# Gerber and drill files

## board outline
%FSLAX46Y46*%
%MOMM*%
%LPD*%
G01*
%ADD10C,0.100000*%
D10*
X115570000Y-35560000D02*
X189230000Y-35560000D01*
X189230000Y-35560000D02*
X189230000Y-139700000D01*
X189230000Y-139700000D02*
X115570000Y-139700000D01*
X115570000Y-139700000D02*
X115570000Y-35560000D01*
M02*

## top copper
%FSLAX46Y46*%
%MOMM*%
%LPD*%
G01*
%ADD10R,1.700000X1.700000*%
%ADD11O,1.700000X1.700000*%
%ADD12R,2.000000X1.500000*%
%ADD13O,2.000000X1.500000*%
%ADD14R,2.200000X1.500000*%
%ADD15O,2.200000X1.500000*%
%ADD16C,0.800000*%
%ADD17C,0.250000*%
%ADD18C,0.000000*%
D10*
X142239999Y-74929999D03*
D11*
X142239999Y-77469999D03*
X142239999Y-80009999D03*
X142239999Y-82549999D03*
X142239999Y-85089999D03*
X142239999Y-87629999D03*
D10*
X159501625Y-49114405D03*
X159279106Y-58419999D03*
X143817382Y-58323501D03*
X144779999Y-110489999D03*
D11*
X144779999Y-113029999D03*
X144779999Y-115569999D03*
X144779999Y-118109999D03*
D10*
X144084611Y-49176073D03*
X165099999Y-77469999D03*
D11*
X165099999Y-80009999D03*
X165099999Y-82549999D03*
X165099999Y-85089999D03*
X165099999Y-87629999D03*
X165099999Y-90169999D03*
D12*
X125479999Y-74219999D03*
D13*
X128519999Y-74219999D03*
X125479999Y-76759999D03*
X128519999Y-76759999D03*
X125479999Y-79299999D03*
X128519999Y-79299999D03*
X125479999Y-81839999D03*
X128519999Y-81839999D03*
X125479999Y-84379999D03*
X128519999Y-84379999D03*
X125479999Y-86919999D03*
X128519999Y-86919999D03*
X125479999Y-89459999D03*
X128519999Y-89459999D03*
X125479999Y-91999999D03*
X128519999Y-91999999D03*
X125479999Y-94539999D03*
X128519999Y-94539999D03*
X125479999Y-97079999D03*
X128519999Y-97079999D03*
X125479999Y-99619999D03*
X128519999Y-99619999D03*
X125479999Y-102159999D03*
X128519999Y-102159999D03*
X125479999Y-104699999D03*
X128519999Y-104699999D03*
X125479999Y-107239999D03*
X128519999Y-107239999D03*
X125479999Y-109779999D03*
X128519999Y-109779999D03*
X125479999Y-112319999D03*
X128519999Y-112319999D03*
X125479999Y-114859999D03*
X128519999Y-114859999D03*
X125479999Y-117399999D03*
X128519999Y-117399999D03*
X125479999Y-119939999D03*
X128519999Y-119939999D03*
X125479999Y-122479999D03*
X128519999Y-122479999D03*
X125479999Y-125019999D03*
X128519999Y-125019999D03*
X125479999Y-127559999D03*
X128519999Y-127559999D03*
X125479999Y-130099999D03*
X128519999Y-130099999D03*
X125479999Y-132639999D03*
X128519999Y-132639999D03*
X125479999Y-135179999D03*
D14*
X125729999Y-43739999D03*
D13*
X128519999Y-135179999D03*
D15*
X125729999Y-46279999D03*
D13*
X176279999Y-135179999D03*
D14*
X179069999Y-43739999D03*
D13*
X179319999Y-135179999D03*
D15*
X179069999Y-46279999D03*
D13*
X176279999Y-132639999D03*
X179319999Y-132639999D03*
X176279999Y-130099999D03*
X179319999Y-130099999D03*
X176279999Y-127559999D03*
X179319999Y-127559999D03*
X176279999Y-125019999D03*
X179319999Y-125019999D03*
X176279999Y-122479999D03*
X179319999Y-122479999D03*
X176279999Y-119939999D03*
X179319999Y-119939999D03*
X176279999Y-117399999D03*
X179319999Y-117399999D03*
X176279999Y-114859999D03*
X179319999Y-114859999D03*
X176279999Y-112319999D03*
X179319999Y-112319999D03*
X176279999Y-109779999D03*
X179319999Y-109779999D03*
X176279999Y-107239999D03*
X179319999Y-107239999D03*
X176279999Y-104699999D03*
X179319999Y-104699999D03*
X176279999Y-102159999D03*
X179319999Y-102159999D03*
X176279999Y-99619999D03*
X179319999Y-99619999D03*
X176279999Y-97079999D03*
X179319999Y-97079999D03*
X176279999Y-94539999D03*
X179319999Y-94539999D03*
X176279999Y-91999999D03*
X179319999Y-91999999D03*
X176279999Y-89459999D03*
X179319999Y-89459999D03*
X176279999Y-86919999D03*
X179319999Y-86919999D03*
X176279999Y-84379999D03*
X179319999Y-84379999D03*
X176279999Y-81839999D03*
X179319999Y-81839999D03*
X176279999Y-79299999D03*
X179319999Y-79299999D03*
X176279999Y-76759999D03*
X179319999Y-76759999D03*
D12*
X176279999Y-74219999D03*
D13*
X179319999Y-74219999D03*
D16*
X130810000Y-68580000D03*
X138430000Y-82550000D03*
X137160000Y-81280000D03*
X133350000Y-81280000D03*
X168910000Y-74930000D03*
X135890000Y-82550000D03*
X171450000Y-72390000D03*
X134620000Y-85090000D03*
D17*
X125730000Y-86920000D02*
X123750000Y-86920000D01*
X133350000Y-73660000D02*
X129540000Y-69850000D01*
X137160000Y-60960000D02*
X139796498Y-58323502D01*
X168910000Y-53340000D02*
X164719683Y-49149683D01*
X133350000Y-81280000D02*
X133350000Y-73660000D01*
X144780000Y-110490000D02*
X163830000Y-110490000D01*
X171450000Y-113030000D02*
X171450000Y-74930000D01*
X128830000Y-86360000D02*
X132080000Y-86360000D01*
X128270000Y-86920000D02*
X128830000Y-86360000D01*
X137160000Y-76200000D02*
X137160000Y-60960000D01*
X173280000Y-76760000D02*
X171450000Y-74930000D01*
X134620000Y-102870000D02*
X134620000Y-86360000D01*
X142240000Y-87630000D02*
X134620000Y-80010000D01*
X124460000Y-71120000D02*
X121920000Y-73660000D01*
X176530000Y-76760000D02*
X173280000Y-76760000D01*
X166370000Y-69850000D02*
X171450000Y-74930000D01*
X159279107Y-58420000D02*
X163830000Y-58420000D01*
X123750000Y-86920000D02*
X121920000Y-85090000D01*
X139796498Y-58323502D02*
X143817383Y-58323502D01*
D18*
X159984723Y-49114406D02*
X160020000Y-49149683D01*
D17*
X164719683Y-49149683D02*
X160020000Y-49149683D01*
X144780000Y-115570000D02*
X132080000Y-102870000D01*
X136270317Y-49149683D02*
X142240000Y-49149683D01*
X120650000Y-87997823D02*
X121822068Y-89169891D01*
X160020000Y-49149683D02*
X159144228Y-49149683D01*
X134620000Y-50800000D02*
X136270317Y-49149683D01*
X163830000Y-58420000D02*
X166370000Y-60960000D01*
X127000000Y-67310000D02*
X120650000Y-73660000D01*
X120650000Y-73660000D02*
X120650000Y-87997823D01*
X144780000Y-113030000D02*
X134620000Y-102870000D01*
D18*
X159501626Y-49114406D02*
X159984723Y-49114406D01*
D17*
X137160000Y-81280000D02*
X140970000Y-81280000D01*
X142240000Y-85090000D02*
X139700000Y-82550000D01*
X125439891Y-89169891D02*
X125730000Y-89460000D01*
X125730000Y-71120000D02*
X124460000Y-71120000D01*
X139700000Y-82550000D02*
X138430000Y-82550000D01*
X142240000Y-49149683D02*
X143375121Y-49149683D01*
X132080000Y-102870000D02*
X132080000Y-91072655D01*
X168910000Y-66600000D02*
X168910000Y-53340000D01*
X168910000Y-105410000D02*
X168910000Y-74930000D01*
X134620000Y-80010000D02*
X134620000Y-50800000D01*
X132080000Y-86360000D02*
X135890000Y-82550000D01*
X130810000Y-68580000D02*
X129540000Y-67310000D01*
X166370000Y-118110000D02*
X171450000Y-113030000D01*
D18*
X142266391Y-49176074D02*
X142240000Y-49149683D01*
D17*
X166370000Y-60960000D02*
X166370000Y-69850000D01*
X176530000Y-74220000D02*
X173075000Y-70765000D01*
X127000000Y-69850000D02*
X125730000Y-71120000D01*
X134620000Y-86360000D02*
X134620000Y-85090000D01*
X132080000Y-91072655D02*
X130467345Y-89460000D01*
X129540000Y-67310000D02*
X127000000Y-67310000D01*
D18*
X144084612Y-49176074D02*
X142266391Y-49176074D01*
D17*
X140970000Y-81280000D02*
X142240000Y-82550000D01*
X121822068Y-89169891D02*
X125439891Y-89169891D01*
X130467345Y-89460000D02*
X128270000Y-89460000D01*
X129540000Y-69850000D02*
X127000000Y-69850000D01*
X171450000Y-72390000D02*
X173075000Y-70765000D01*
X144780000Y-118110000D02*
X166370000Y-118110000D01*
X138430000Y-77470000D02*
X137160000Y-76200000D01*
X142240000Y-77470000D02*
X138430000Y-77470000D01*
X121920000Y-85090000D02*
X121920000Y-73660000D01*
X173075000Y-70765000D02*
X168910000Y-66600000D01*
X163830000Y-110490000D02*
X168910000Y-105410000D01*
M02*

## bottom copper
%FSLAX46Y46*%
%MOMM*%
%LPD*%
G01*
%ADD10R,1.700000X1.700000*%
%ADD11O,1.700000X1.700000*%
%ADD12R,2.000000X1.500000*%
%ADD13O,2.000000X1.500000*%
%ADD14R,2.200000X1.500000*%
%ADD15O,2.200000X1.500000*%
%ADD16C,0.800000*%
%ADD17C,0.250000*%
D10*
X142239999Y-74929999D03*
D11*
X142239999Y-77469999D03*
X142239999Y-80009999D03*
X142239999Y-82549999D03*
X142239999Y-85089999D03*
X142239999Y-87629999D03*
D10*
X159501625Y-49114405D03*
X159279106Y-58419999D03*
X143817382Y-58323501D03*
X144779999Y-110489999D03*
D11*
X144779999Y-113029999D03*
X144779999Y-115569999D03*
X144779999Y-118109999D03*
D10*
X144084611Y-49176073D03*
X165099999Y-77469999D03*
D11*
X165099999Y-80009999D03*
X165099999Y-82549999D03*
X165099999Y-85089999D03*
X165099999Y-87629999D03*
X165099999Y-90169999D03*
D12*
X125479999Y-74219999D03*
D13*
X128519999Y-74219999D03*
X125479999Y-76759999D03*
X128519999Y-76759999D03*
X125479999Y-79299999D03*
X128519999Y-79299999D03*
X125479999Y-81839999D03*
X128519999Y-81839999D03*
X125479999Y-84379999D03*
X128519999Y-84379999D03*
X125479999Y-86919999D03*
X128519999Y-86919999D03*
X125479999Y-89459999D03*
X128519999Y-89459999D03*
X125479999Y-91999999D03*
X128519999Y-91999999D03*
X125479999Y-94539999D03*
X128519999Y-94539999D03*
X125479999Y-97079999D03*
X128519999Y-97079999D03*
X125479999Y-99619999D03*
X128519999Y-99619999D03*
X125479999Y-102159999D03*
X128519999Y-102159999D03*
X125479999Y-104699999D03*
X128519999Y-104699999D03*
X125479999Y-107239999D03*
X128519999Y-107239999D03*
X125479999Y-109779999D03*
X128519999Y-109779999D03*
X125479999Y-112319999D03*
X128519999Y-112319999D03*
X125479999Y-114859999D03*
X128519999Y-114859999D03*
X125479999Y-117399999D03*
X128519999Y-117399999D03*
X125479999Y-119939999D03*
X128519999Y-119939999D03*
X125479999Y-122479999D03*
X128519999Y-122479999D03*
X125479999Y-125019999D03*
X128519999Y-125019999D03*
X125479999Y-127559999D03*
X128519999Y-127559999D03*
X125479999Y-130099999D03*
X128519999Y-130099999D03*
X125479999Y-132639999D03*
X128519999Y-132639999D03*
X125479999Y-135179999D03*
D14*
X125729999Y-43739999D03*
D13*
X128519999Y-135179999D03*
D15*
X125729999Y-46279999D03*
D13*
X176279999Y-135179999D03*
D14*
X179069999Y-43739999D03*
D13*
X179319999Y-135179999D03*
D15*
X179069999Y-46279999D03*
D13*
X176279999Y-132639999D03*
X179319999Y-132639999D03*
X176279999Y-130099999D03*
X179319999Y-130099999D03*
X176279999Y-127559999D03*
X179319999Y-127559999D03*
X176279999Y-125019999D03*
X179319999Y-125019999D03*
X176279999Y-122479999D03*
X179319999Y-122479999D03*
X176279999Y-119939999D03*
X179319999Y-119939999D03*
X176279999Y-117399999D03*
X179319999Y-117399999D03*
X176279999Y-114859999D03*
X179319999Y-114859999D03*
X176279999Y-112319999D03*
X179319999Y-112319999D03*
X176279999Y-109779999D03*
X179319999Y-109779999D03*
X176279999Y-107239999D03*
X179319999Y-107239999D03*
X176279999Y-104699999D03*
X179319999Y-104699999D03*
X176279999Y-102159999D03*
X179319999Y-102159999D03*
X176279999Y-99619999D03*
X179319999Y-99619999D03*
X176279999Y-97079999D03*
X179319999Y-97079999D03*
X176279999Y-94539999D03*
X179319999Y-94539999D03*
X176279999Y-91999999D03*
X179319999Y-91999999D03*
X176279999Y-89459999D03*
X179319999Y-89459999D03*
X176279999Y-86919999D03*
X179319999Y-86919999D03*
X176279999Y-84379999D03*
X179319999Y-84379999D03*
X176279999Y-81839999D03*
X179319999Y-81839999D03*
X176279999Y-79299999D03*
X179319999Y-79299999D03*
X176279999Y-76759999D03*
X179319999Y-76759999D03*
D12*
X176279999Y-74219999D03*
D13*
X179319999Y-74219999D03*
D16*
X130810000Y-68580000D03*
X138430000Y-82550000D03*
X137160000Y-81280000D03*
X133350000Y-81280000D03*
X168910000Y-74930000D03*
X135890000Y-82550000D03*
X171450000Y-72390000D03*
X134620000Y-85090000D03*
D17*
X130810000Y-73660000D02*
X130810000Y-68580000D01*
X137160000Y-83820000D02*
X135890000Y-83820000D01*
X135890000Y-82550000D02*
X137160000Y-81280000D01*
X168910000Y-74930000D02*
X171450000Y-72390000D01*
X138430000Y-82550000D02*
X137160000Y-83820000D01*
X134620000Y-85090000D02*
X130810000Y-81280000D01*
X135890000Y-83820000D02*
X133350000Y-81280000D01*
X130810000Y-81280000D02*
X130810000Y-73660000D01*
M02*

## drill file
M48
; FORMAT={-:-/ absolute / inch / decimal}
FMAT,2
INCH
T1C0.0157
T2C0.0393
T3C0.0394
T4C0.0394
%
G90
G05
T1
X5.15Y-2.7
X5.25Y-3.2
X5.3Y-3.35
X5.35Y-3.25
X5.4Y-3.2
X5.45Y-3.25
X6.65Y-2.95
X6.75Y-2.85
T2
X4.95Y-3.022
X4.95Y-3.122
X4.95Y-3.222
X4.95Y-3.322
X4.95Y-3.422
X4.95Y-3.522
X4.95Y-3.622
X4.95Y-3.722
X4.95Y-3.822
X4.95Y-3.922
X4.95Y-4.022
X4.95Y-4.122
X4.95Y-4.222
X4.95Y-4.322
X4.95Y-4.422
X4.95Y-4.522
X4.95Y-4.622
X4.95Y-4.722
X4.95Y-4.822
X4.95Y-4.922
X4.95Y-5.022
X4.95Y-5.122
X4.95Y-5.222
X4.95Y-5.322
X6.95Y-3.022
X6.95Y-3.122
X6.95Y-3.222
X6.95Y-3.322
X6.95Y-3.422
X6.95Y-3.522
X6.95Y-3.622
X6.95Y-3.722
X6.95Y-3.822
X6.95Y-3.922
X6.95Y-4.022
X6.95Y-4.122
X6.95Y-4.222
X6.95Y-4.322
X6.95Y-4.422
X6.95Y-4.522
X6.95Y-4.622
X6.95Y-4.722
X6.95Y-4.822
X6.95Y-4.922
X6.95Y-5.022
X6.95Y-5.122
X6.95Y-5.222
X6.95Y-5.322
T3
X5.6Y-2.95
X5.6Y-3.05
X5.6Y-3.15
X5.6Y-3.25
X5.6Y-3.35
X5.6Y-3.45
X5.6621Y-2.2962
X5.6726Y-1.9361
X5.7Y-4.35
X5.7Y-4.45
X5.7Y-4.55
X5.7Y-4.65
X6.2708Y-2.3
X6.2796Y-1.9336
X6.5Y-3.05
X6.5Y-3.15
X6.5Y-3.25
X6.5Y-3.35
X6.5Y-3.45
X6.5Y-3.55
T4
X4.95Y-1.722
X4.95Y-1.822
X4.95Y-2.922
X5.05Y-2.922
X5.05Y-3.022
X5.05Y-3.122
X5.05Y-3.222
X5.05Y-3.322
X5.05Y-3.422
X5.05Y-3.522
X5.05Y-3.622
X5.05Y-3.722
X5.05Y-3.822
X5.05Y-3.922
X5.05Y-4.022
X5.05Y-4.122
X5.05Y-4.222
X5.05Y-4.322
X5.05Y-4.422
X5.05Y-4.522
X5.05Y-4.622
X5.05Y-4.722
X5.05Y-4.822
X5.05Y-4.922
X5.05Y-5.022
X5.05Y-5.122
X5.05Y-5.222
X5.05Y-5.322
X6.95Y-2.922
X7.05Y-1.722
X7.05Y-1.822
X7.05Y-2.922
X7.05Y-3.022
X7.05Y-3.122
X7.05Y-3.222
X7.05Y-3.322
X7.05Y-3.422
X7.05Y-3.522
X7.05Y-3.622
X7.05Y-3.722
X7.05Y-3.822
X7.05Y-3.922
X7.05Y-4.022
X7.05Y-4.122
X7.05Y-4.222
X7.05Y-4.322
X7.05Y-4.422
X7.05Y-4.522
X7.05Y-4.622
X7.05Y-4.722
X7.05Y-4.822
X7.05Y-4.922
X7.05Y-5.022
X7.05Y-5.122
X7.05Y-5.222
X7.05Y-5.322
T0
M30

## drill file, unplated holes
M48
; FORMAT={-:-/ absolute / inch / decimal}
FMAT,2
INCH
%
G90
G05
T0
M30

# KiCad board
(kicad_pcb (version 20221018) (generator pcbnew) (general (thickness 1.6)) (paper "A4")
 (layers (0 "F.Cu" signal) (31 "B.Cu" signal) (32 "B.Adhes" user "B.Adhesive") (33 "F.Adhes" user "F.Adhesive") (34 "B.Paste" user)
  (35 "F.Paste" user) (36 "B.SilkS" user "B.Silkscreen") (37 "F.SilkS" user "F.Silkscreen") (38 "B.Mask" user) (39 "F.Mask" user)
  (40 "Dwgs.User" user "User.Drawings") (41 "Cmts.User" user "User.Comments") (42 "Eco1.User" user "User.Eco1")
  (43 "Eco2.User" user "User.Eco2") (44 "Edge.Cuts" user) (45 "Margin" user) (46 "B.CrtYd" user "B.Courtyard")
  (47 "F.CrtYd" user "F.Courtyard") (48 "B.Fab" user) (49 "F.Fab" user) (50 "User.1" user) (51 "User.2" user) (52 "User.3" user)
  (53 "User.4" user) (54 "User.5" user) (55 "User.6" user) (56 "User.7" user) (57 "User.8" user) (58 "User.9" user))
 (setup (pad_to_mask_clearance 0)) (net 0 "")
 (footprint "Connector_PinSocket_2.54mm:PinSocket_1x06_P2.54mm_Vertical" (layer "F.Cu") (at 142.24 74.93)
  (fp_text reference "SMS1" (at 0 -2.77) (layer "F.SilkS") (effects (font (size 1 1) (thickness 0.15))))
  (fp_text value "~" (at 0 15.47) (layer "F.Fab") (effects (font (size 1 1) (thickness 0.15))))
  (pad "1" thru_hole rect (at 0 0) (size 1.7 1.7) (drill 1) (layers "*.Cu" "*.Mask"))
  (pad "2" thru_hole oval (at 0 2.54) (size 1.7 1.7) (drill 1) (layers "*.Cu" "*.Mask"))
  (pad "3" thru_hole oval (at 0 5.08) (size 1.7 1.7) (drill 1) (layers "*.Cu" "*.Mask"))
  (pad "4" thru_hole oval (at 0 7.62) (size 1.7 1.7) (drill 1) (layers "*.Cu" "*.Mask"))
  (pad "5" thru_hole oval (at 0 10.16) (size 1.7 1.7) (drill 1) (layers "*.Cu" "*.Mask"))
  (pad "6" thru_hole oval (at 0 12.7) (size 1.7 1.7) (drill 1) (layers "*.Cu" "*.Mask")))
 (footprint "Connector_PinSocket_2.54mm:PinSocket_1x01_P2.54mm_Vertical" (layer "F.Cu") (at 159.501626 49.114406 180)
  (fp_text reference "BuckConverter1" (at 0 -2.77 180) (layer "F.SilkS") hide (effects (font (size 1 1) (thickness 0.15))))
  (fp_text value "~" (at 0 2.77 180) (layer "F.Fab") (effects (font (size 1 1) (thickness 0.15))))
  (pad "1" thru_hole rect (at 0 0 180) (size 1.7 1.7) (drill 1) (layers "*.Cu" "*.Mask")))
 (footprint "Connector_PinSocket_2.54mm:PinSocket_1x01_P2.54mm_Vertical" (layer "F.Cu") (at 159.279107 58.42 180)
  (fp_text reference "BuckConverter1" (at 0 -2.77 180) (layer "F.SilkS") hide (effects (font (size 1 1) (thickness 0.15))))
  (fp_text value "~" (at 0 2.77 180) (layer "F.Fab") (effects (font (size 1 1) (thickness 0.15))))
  (pad "1" thru_hole rect (at 0 0 180) (size 1.7 1.7) (drill 1) (layers "*.Cu" "*.Mask")))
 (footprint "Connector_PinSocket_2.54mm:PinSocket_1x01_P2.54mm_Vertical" (layer "F.Cu") (at 143.817383 58.323502 180)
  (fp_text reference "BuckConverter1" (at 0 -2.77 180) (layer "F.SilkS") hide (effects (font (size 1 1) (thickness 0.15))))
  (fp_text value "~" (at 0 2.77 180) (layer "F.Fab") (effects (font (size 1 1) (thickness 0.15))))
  (pad "1" thru_hole rect (at 0 0 180) (size 1.7 1.7) (drill 1) (layers "*.Cu" "*.Mask")))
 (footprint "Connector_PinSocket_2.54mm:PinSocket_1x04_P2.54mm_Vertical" (layer "F.Cu") (at 144.78 110.49)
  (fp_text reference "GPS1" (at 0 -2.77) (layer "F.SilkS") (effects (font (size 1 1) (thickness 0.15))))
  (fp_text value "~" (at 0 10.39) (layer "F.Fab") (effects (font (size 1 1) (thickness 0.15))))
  (pad "1" thru_hole rect (at 0 0) (size 1.7 1.7) (drill 1) (layers "*.Cu" "*.Mask"))
  (pad "2" thru_hole oval (at 0 2.54) (size 1.7 1.7) (drill 1) (layers "*.Cu" "*.Mask"))
  (pad "3" thru_hole oval (at 0 5.08) (size 1.7 1.7) (drill 1) (layers "*.Cu" "*.Mask"))
  (pad "4" thru_hole oval (at 0 7.62) (size 1.7 1.7) (drill 1) (layers "*.Cu" "*.Mask")))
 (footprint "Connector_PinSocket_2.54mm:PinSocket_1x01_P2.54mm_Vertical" (layer "F.Cu") (at 144.084612 49.176074 180)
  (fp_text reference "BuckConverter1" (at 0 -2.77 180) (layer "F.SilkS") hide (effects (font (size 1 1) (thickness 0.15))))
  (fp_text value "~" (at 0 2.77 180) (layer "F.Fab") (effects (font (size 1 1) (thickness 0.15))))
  (pad "1" thru_hole rect (at 0 0 180) (size 1.7 1.7) (drill 1) (layers "*.Cu" "*.Mask")))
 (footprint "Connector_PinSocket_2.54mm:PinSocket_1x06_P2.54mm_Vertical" (layer "F.Cu") (at 165.1 77.47)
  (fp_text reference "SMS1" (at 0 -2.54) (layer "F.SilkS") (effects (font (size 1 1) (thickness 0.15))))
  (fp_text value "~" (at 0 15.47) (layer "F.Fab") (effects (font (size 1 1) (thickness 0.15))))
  (pad "1" thru_hole rect (at 0 0) (size 1.7 1.7) (drill 1) (layers "*.Cu" "*.Mask"))
  (pad "2" thru_hole oval (at 0 2.54) (size 1.7 1.7) (drill 1) (layers "*.Cu" "*.Mask"))
  (pad "3" thru_hole oval (at 0 5.08) (size 1.7 1.7) (drill 1) (layers "*.Cu" "*.Mask"))
  (pad "4" thru_hole oval (at 0 7.62) (size 1.7 1.7) (drill 1) (layers "*.Cu" "*.Mask"))
  (pad "5" thru_hole oval (at 0 10.16) (size 1.7 1.7) (drill 1) (layers "*.Cu" "*.Mask"))
  (pad "6" thru_hole oval (at 0 12.7) (size 1.7 1.7) (drill 1) (layers "*.Cu" "*.Mask")))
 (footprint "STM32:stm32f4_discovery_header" (layer "F.Cu") (at 152.4 88.9 90)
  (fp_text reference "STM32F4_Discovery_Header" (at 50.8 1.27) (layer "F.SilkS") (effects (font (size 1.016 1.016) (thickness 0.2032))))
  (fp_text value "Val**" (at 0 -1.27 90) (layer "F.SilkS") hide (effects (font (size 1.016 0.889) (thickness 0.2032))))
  (pad "1" thru_hole rect (at 14.68 -26.67 90) (size 1.5 2) (drill 1.00076 (offset 0 -0.25)) (layers "*.Cu" "*.Mask" "F.SilkS"))
  (pad "2" thru_hole oval (at 14.68 -24.13 90) (size 1.5 2) (drill 1.00076 (offset 0 0.25)) (layers "*.Cu" "*.Mask" "F.SilkS"))
  (pad "3" thru_hole oval (at 12.14 -26.67 90) (size 1.5 2) (drill 0.99822 (offset 0 -0.25)) (layers "*.Cu" "*.Mask" "F.SilkS"))
  (pad "4" thru_hole oval (at 12.14 -24.13 90) (size 1.5 2) (drill 1.00076 (offset 0 0.25)) (layers "*.Cu" "*.Mask" "F.SilkS"))
  (pad "5" thru_hole oval (at 9.6 -26.67 90) (size 1.5 2) (drill 0.99822 (offset 0 -0.25)) (layers "*.Cu" "*.Mask" "F.SilkS"))
  (pad "6" thru_hole oval (at 9.6 -24.13 90) (size 1.5 2) (drill 1.00076 (offset 0 0.25)) (layers "*.Cu" "*.Mask" "F.SilkS"))
  (pad "7" thru_hole oval (at 7.06 -26.67 90) (size 1.5 2) (drill 0.99822 (offset 0 -0.25)) (layers "*.Cu" "*.Mask" "F.SilkS"))
  (pad "8" thru_hole oval (at 7.06 -24.13 90) (size 1.5 2) (drill 1.00076 (offset 0 0.25)) (layers "*.Cu" "*.Mask" "F.SilkS"))
  (pad "9" thru_hole oval (at 4.52 -26.67 90) (size 1.5 2) (drill 0.99822 (offset 0 -0.25)) (layers "*.Cu" "*.Mask" "F.SilkS"))
  (pad "10" thru_hole oval (at 4.52 -24.13 90) (size 1.5 2) (drill 1.00076 (offset 0 0.25)) (layers "*.Cu" "*.Mask" "F.SilkS"))
  (pad "11" thru_hole oval (at 1.98 -26.67 90) (size 1.5 2) (drill 0.99822 (offset 0 -0.25)) (layers "*.Cu" "*.Mask" "F.SilkS"))
  (pad "12" thru_hole oval (at 1.98 -24.13 90) (size 1.5 2) (drill 1.00076 (offset 0 0.25)) (layers "*.Cu" "*.Mask" "F.SilkS"))
  (pad "13" thru_hole oval (at -0.56 -26.67 90) (size 1.5 2) (drill 0.99822 (offset 0 -0.25)) (layers "*.Cu" "*.Mask" "F.SilkS"))
  (pad "14" thru_hole oval (at -0.56 -24.13 90) (size 1.5 2) (drill 1.00076 (offset 0 0.25)) (layers "*.Cu" "*.Mask" "F.SilkS"))
  (pad "15" thru_hole oval (at -3.1 -26.67 90) (size 1.5 2) (drill 0.99822 (offset 0 -0.25)) (layers "*.Cu" "*.Mask" "F.SilkS"))
  (pad "16" thru_hole oval (at -3.1 -24.13 90) (size 1.5 2) (drill 1.00076 (offset 0 0.25)) (layers "*.Cu" "*.Mask" "F.SilkS"))
  (pad "17" thru_hole oval (at -5.64 -26.67 90) (size 1.5 2) (drill 0.99822 (offset 0 -0.25)) (layers "*.Cu" "*.Mask" "F.SilkS"))
  (pad "18" thru_hole oval (at -5.64 -24.13 90) (size 1.5 2) (drill 1.00076 (offset 0 0.25)) (layers "*.Cu" "*.Mask" "F.SilkS"))
  (pad "19" thru_hole oval (at -8.18 -26.67 90) (size 1.5 2) (drill 0.99822 (offset 0 -0.25)) (layers "*.Cu" "*.Mask" "F.SilkS"))
  (pad "20" thru_hole oval (at -8.18 -24.13 90) (size 1.5 2) (drill 1.00076 (offset 0 0.25)) (layers "*.Cu" "*.Mask" "F.SilkS"))
  (pad "21" thru_hole oval (at -10.72 -26.67 90) (size 1.5 2) (drill 0.99822 (offset 0 -0.25)) (layers "*.Cu" "*.Mask" "F.SilkS"))
  (pad "22" thru_hole oval (at -10.72 -24.13 90) (size 1.5 2) (drill 1.00076 (offset 0 0.25)) (layers "*.Cu" "*.Mask" "F.SilkS"))
  (pad "23" thru_hole oval (at -13.26 -26.67 90) (size 1.5 2) (drill 0.99822 (offset 0 -0.25)) (layers "*.Cu" "*.Mask" "F.SilkS"))
  (pad "24" thru_hole oval (at -13.26 -24.13 90) (size 1.5 2) (drill 1.00076 (offset 0 0.25)) (layers "*.Cu" "*.Mask" "F.SilkS"))
  (pad "25" thru_hole oval (at -15.8 -26.67 90) (size 1.5 2) (drill 0.99822 (offset 0 -0.25)) (layers "*.Cu" "*.Mask" "F.SilkS"))
  (pad "26" thru_hole oval (at -15.8 -24.13 90) (size 1.5 2) (drill 1.00076 (offset 0 0.25)) (layers "*.Cu" "*.Mask" "F.SilkS"))
  (pad "27" thru_hole oval (at -18.34 -26.67 90) (size 1.5 2) (drill 0.99822 (offset 0 -0.25)) (layers "*.Cu" "*.Mask" "F.SilkS"))
  (pad "28" thru_hole oval (at -18.34 -24.13 90) (size 1.5 2) (drill 1.00076 (offset 0 0.25)) (layers "*.Cu" "*.Mask" "F.SilkS"))
  (pad "29" thru_hole oval (at -20.88 -26.67 90) (size 1.5 2) (drill 0.99822 (offset 0 -0.25)) (layers "*.Cu" "*.Mask" "F.SilkS"))
  (pad "30" thru_hole oval (at -20.88 -24.13 90) (size 1.5 2) (drill 1.00076 (offset 0 0.25)) (layers "*.Cu" "*.Mask" "F.SilkS"))
  (pad "31" thru_hole oval (at -23.42 -26.67 90) (size 1.5 2) (drill 0.99822 (offset 0 -0.25)) (layers "*.Cu" "*.Mask" "F.SilkS"))
  (pad "32" thru_hole oval (at -23.42 -24.13 90) (size 1.5 2) (drill 1.00076 (offset 0 0.25)) (layers "*.Cu" "*.Mask" "F.SilkS"))
  (pad "33" thru_hole oval (at -25.96 -26.67 90) (size 1.5 2) (drill 0.99822 (offset 0 -0.25)) (layers "*.Cu" "*.Mask" "F.SilkS"))
  (pad "34" thru_hole oval (at -25.96 -24.13 90) (size 1.5 2) (drill 1.00076 (offset 0 0.25)) (layers "*.Cu" "*.Mask" "F.SilkS"))
  (pad "35" thru_hole oval (at -28.5 -26.67 90) (size 1.5 2) (drill 0.99822 (offset 0 -0.25)) (layers "*.Cu" "*.Mask" "F.SilkS"))
  (pad "36" thru_hole oval (at -28.5 -24.13 90) (size 1.5 2) (drill 1.00076 (offset 0 0.25)) (layers "*.Cu" "*.Mask" "F.SilkS"))
  (pad "37" thru_hole oval (at -31.04 -26.67 90) (size 1.5 2) (drill 0.99822 (offset 0 -0.25)) (layers "*.Cu" "*.Mask" "F.SilkS"))
  (pad "38" thru_hole oval (at -31.04 -24.13 90) (size 1.5 2) (drill 1.00076 (offset 0 0.25)) (layers "*.Cu" "*.Mask" "F.SilkS"))
  (pad "39" thru_hole oval (at -33.58 -26.67 90) (size 1.5 2) (drill 0.99822 (offset 0 -0.25)) (layers "*.Cu" "*.Mask" "F.SilkS"))
  (pad "40" thru_hole oval (at -33.58 -24.13 90) (size 1.5 2) (drill 1.00076 (offset 0 0.25)) (layers "*.Cu" "*.Mask" "F.SilkS"))
  (pad "41" thru_hole oval (at -36.12 -26.67 90) (size 1.5 2) (drill 0.99822 (offset 0 -0.25)) (layers "*.Cu" "*.Mask" "F.SilkS"))
  (pad "42" thru_hole oval (at -36.12 -24.13 90) (size 1.5 2) (drill 1.00076 (offset 0 0.25)) (layers "*.Cu" "*.Mask" "F.SilkS"))
  (pad "43" thru_hole oval (at -38.66 -26.67 90) (size 1.5 2) (drill 0.99822 (offset 0 -0.25)) (layers "*.Cu" "*.Mask" "F.SilkS"))
  (pad "44" thru_hole oval (at -38.66 -24.13 90) (size 1.5 2) (drill 1.00076 (offset 0 0.25)) (layers "*.Cu" "*.Mask" "F.SilkS"))
  (pad "45" thru_hole oval (at -41.2 -26.67 90) (size 1.5 2) (drill 0.99822 (offset 0 -0.25)) (layers "*.Cu" "*.Mask" "F.SilkS"))
  (pad "46" thru_hole oval (at -41.2 -24.13 90) (size 1.5 2) (drill 1.00076 (offset 0 0.25)) (layers "*.Cu" "*.Mask" "F.SilkS"))
  (pad "47" thru_hole oval (at -43.74 -26.67 90) (size 1.5 2) (drill 0.99822 (offset 0 -0.25)) (layers "*.Cu" "*.Mask" "F.SilkS"))
  (pad "48" thru_hole oval (at -43.74 -24.13 90) (size 1.5 2) (drill 1.00076 (offset 0 0.25)) (layers "*.Cu" "*.Mask" "F.SilkS"))
  (pad "49" thru_hole oval (at -46.28 -26.67 90) (size 1.5 2) (drill 0.99822 (offset 0 -0.25)) (layers "*.Cu" "*.Mask" "F.SilkS"))
  (pad "49" thru_hole rect (at 45.16 -26.67 90) (size 1.5 2.2) (drill 1.00076) (layers "*.Cu" "*.Mask" "F.SilkS"))
  (pad "50" thru_hole oval (at -46.28 -24.13 90) (size 1.5 2) (drill 1.00076 (offset 0 0.25)) (layers "*.Cu" "*.Mask" "F.SilkS"))
  (pad "50" thru_hole oval (at 42.62 -26.67 90) (size 1.5 2.2) (drill 1.00076) (layers "*.Cu" "*.Mask" "F.SilkS"))
  (pad "51" thru_hole oval (at -46.28 24.13 90) (size 1.5 2) (drill 0.99822 (offset 0 -0.25)) (layers "*.Cu" "*.Mask" "F.SilkS"))
  (pad "51" thru_hole rect (at 45.16 26.67 90) (size 1.5 2.2) (drill 1.00076) (layers "*.Cu" "*.Mask" "F.SilkS"))
  (pad "52" thru_hole oval (at -46.28 26.67 90) (size 1.5 2) (drill 1.00076 (offset 0 0.25)) (layers "*.Cu" "*.Mask" "F.SilkS"))
  (pad "52" thru_hole oval (at 42.62 26.67 90) (size 1.5 2.2) (drill 1.00076) (layers "*.Cu" "*.Mask" "F.SilkS"))
  (pad "53" thru_hole oval (at -43.74 24.13 90) (size 1.5 2) (drill 0.99822 (offset 0 -0.25)) (layers "*.Cu" "*.Mask" "F.SilkS"))
  (pad "54" thru_hole oval (at -43.74 26.67 90) (size 1.5 2) (drill 1.00076 (offset 0 0.25)) (layers "*.Cu" "*.Mask" "F.SilkS"))
  (pad "55" thru_hole oval (at -41.2 24.13 90) (size 1.5 2) (drill 0.99822 (offset 0 -0.25)) (layers "*.Cu" "*.Mask" "F.SilkS"))
  (pad "56" thru_hole oval (at -41.2 26.67 90) (size 1.5 2) (drill 1.00076 (offset 0 0.25)) (layers "*.Cu" "*.Mask" "F.SilkS"))
  (pad "57" thru_hole oval (at -38.66 24.13 90) (size 1.5 2) (drill 0.99822 (offset 0 -0.25)) (layers "*.Cu" "*.Mask" "F.SilkS"))
  (pad "58" thru_hole oval (at -38.66 26.67 90) (size 1.5 2) (drill 1.00076 (offset 0 0.25)) (layers "*.Cu" "*.Mask" "F.SilkS"))
  (pad "59" thru_hole oval (at -36.12 24.13 90) (size 1.5 2) (drill 0.99822 (offset 0 -0.25)) (layers "*.Cu" "*.Mask" "F.SilkS"))
  (pad "60" thru_hole oval (at -36.12 26.67 90) (size 1.5 2) (drill 1.00076 (offset 0 0.25)) (layers "*.Cu" "*.Mask" "F.SilkS"))
  (pad "61" thru_hole oval (at -33.58 24.13 90) (size 1.5 2) (drill 0.99822 (offset 0 -0.25)) (layers "*.Cu" "*.Mask" "F.SilkS"))
  (pad "62" thru_hole oval (at -33.58 26.67 90) (size 1.5 2) (drill 1.00076 (offset 0 0.25)) (layers "*.Cu" "*.Mask" "F.SilkS"))
  (pad "63" thru_hole oval (at -31.04 24.13 90) (size 1.5 2) (drill 0.99822 (offset 0 -0.25)) (layers "*.Cu" "*.Mask" "F.SilkS"))
  (pad "64" thru_hole oval (at -31.04 26.67 90) (size 1.5 2) (drill 1.00076 (offset 0 0.25)) (layers "*.Cu" "*.Mask" "F.SilkS"))
  (pad "65" thru_hole oval (at -28.5 24.13 90) (size 1.5 2) (drill 0.99822 (offset 0 -0.25)) (layers "*.Cu" "*.Mask" "F.SilkS"))
  (pad "66" thru_hole oval (at -28.5 26.67 90) (size 1.5 2) (drill 1.00076 (offset 0 0.25)) (layers "*.Cu" "*.Mask" "F.SilkS"))
  (pad "67" thru_hole oval (at -25.96 24.13 90) (size 1.5 2) (drill 0.99822 (offset 0 -0.25)) (layers "*.Cu" "*.Mask" "F.SilkS"))
  (pad "68" thru_hole oval (at -25.96 26.67 90) (size 1.5 2) (drill 1.00076 (offset 0 0.25)) (layers "*.Cu" "*.Mask" "F.SilkS"))
  (pad "69" thru_hole oval (at -23.42 24.13 90) (size 1.5 2) (drill 0.99822 (offset 0 -0.25)) (layers "*.Cu" "*.Mask" "F.SilkS"))
  (pad "70" thru_hole oval (at -23.42 26.67 90) (size 1.5 2) (drill 1.00076 (offset 0 0.25)) (layers "*.Cu" "*.Mask" "F.SilkS"))
  (pad "71" thru_hole oval (at -20.88 24.13 90) (size 1.5 2) (drill 0.99822 (offset 0 -0.25)) (layers "*.Cu" "*.Mask" "F.SilkS"))
  (pad "72" thru_hole oval (at -20.88 26.67 90) (size 1.5 2) (drill 1.00076 (offset 0 0.25)) (layers "*.Cu" "*.Mask" "F.SilkS"))
  (pad "73" thru_hole oval (at -18.34 24.13 90) (size 1.5 2) (drill 0.99822 (offset 0 -0.25)) (layers "*.Cu" "*.Mask" "F.SilkS"))
  (pad "74" thru_hole oval (at -18.34 26.67 90) (size 1.5 2) (drill 1.00076 (offset 0 0.25)) (layers "*.Cu" "*.Mask" "F.SilkS"))
  (pad "75" thru_hole oval (at -15.8 24.13 90) (size 1.5 2) (drill 0.99822 (offset 0 -0.25)) (layers "*.Cu" "*.Mask" "F.SilkS"))
  (pad "76" thru_hole oval (at -15.8 26.67 90) (size 1.5 2) (drill 1.00076 (offset 0 0.25)) (layers "*.Cu" "*.Mask" "F.SilkS"))
  (pad "77" thru_hole oval (at -13.26 24.13 90) (size 1.5 2) (drill 0.99822 (offset 0 -0.25)) (layers "*.Cu" "*.Mask" "F.SilkS"))
  (pad "78" thru_hole oval (at -13.26 26.67 90) (size 1.5 2) (drill 1.00076 (offset 0 0.25)) (layers "*.Cu" "*.Mask" "F.SilkS"))
  (pad "79" thru_hole oval (at -10.72 24.13 90) (size 1.5 2) (drill 0.99822 (offset 0 -0.25)) (layers "*.Cu" "*.Mask" "F.SilkS"))
  (pad "80" thru_hole oval (at -10.72 26.67 90) (size 1.5 2) (drill 1.00076 (offset 0 0.25)) (layers "*.Cu" "*.Mask" "F.SilkS"))
  (pad "81" thru_hole oval (at -8.18 24.13 90) (size 1.5 2) (drill 0.99822 (offset 0 -0.25)) (layers "*.Cu" "*.Mask" "F.SilkS"))
  (pad "82" thru_hole oval (at -8.18 26.67 90) (size 1.5 2) (drill 1.00076 (offset 0 0.25)) (layers "*.Cu" "*.Mask" "F.SilkS"))
  (pad "83" thru_hole oval (at -5.64 24.13 90) (size 1.5 2) (drill 0.99822 (offset 0 -0.25)) (layers "*.Cu" "*.Mask" "F.SilkS"))
  (pad "84" thru_hole oval (at -5.64 26.67 90) (size 1.5 2) (drill 1.00076 (offset 0 0.25)) (layers "*.Cu" "*.Mask" "F.SilkS"))
  (pad "85" thru_hole oval (at -3.1 24.13 90) (size 1.5 2) (drill 0.99822 (offset 0 -0.25)) (layers "*.Cu" "*.Mask" "F.SilkS"))
  (pad "86" thru_hole oval (at -3.1 26.67 90) (size 1.5 2) (drill 1.00076 (offset 0 0.25)) (layers "*.Cu" "*.Mask" "F.SilkS"))
  (pad "87" thru_hole oval (at -0.56 24.13 90) (size 1.5 2) (drill 0.99822 (offset 0 -0.25)) (layers "*.Cu" "*.Mask" "F.SilkS"))
  (pad "88" thru_hole oval (at -0.56 26.67 90) (size 1.5 2) (drill 1.00076 (offset 0 0.25)) (layers "*.Cu" "*.Mask" "F.SilkS"))
  (pad "89" thru_hole oval (at 1.98 24.13 90) (size 1.5 2) (drill 0.99822 (offset 0 -0.25)) (layers "*.Cu" "*.Mask" "F.SilkS"))
  (pad "90" thru_hole oval (at 1.98 26.67 90) (size 1.5 2) (drill 1.00076 (offset 0 0.25)) (layers "*.Cu" "*.Mask" "F.SilkS"))
  (pad "91" thru_hole oval (at 4.52 24.13 90) (size 1.5 2) (drill 0.99822 (offset 0 -0.25)) (layers "*.Cu" "*.Mask" "F.SilkS"))
  (pad "92" thru_hole oval (at 4.52 26.67 90) (size 1.5 2) (drill 1.00076 (offset 0 0.25)) (layers "*.Cu" "*.Mask" "F.SilkS"))
  (pad "93" thru_hole oval (at 7.06 24.13 90) (size 1.5 2) (drill 0.99822 (offset 0 -0.25)) (layers "*.Cu" "*.Mask" "F.SilkS"))
  (pad "94" thru_hole oval (at 7.06 26.67 90) (size 1.5 2) (drill 1.00076 (offset 0 0.25)) (layers "*.Cu" "*.Mask" "F.SilkS"))
  (pad "95" thru_hole oval (at 9.6 24.13 90) (size 1.5 2) (drill 0.99822 (offset 0 -0.25)) (layers "*.Cu" "*.Mask" "F.SilkS"))
  (pad "96" thru_hole oval (at 9.6 26.67 90) (size 1.5 2) (drill 1.00076 (offset 0 0.25)) (layers "*.Cu" "*.Mask" "F.SilkS"))
  (pad "97" thru_hole oval (at 12.14 24.13 90) (size 1.5 2) (drill 0.99822 (offset 0 -0.25)) (layers "*.Cu" "*.Mask" "F.SilkS"))
  (pad "98" thru_hole oval (at 12.14 26.67 90) (size 1.5 2) (drill 1.00076 (offset 0 0.25)) (layers "*.Cu" "*.Mask" "F.SilkS"))
  (pad "99" thru_hole rect (at 14.68 24.13 90) (size 1.5 2) (drill 1.00076 (offset 0 -0.25)) (layers "*.Cu" "*.Mask" "F.SilkS"))
  (pad "100" thru_hole oval (at 14.68 26.67 90) (size 1.5 2) (drill 1.00076 (offset 0 0.25)) (layers "*.Cu" "*.Mask" "F.SilkS")))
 (gr_rect (start 115.57 35.56) (end 189.23 139.7) (stroke (width 0.1) (type default)) (fill none) (layer "Edge.Cuts"))
 (segment (start 125.73 86.92) (end 123.75 86.92) (width 0.25) (layer "F.Cu") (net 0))
 (segment (start 133.35 73.66) (end 129.54 69.85) (width 0.25) (layer "F.Cu") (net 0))
 (segment (start 137.16 60.96) (end 139.796498 58.323502) (width 0.25) (layer "F.Cu") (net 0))
 (segment (start 168.91 53.34) (end 164.719683 49.149683) (width 0.25) (layer "F.Cu") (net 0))
 (segment (start 133.35 81.28) (end 133.35 73.66) (width 0.25) (layer "F.Cu") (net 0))
 (segment (start 144.78 110.49) (end 163.83 110.49) (width 0.25) (layer "F.Cu") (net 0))
 (segment (start 171.45 113.03) (end 171.45 74.93) (width 0.25) (layer "F.Cu") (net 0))
 (segment (start 128.83 86.36) (end 132.08 86.36) (width 0.25) (layer "F.Cu") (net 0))
 (segment (start 128.27 86.92) (end 128.83 86.36) (width 0.25) (layer "F.Cu") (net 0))
 (segment (start 137.16 76.2) (end 137.16 60.96) (width 0.25) (layer "F.Cu") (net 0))
 (segment (start 173.28 76.76) (end 171.45 74.93) (width 0.25) (layer "F.Cu") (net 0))
 (segment (start 134.62 102.87) (end 134.62 86.36) (width 0.25) (layer "F.Cu") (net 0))
 (segment (start 142.24 87.63) (end 134.62 80.01) (width 0.25) (layer "F.Cu") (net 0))
 (segment (start 124.46 71.12) (end 121.92 73.66) (width 0.25) (layer "F.Cu") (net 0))
 (segment (start 176.53 76.76) (end 173.28 76.76) (width 0.25) (layer "F.Cu") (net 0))
 (segment (start 166.37 69.85) (end 171.45 74.93) (width 0.25) (layer "F.Cu") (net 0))
 (segment (start 159.279107 58.42) (end 163.83 58.42) (width 0.25) (layer "F.Cu") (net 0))
 (segment (start 123.75 86.92) (end 121.92 85.09) (width 0.25) (layer "F.Cu") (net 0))
 (segment (start 139.796498 58.323502) (end 143.817383 58.323502) (width 0.25) (layer "F.Cu") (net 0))
 (segment (start 159.984723 49.114406) (end 160.02 49.149683) (width 0) (layer "F.Cu") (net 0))
 (segment (start 164.719683 49.149683) (end 160.02 49.149683) (width 0.25) (layer "F.Cu") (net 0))
 (segment (start 144.78 115.57) (end 132.08 102.87) (width 0.25) (layer "F.Cu") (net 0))
 (segment (start 136.270317 49.149683) (end 142.24 49.149683) (width 0.25) (layer "F.Cu") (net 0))
 (segment (start 120.65 87.997823) (end 121.822068 89.169891) (width 0.25) (layer "F.Cu") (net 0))
 (segment (start 160.02 49.149683) (end 159.144228 49.149683) (width 0.25) (layer "F.Cu") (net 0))
 (segment (start 134.62 50.8) (end 136.270317 49.149683) (width 0.25) (layer "F.Cu") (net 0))
 (segment (start 163.83 58.42) (end 166.37 60.96) (width 0.25) (layer "F.Cu") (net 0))
 (segment (start 127 67.31) (end 120.65 73.66) (width 0.25) (layer "F.Cu") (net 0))
 (segment (start 120.65 73.66) (end 120.65 87.997823) (width 0.25) (layer "F.Cu") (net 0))
 (segment (start 144.78 113.03) (end 134.62 102.87) (width 0.25) (layer "F.Cu") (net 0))
 (segment (start 159.501626 49.114406) (end 159.984723 49.114406) (width 0) (layer "F.Cu") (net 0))
 (segment (start 137.16 81.28) (end 140.97 81.28) (width 0.25) (layer "F.Cu") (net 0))
 (segment (start 142.24 85.09) (end 139.7 82.55) (width 0.25) (layer "F.Cu") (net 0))
 (segment (start 125.439891 89.169891) (end 125.73 89.46) (width 0.25) (layer "F.Cu") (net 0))
 (segment (start 125.73 71.12) (end 124.46 71.12) (width 0.25) (layer "F.Cu") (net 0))
 (segment (start 139.7 82.55) (end 138.43 82.55) (width 0.25) (layer "F.Cu") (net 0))
 (segment (start 142.24 49.149683) (end 143.375121 49.149683) (width 0.25) (layer "F.Cu") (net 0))
 (segment (start 132.08 102.87) (end 132.08 91.072655) (width 0.25) (layer "F.Cu") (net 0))
 (segment (start 168.91 66.6) (end 168.91 53.34) (width 0.25) (layer "F.Cu") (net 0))
 (segment (start 168.91 105.41) (end 168.91 74.93) (width 0.25) (layer "F.Cu") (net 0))
 (segment (start 134.62 80.01) (end 134.62 50.8) (width 0.25) (layer "F.Cu") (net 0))
 (segment (start 132.08 86.36) (end 135.89 82.55) (width 0.25) (layer "F.Cu") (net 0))
 (segment (start 130.81 68.58) (end 129.54 67.31) (width 0.25) (layer "F.Cu") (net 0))
 (segment (start 166.37 118.11) (end 171.45 113.03) (width 0.25) (layer "F.Cu") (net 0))
 (segment (start 142.266391 49.176074) (end 142.24 49.149683) (width 0) (layer "F.Cu") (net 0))
 (segment (start 166.37 60.96) (end 166.37 69.85) (width 0.25) (layer "F.Cu") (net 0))
 (segment (start 176.53 74.22) (end 173.075 70.765) (width 0.25) (layer "F.Cu") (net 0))
 (segment (start 127 69.85) (end 125.73 71.12) (width 0.25) (layer "F.Cu") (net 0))
 (segment (start 134.62 86.36) (end 134.62 85.09) (width 0.25) (layer "F.Cu") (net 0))
 (segment (start 132.08 91.072655) (end 130.467345 89.46) (width 0.25) (layer "F.Cu") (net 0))
 (segment (start 129.54 67.31) (end 127 67.31) (width 0.25) (layer "F.Cu") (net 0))
 (segment (start 144.084612 49.176074) (end 142.266391 49.176074) (width 0) (layer "F.Cu") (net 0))
 (segment (start 140.97 81.28) (end 142.24 82.55) (width 0.25) (layer "F.Cu") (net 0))
 (segment (start 121.822068 89.169891) (end 125.439891 89.169891) (width 0.25) (layer "F.Cu") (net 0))
 (segment (start 130.467345 89.46) (end 128.27 89.46) (width 0.25) (layer "F.Cu") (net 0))
 (segment (start 129.54 69.85) (end 127 69.85) (width 0.25) (layer "F.Cu") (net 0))
 (segment (start 171.45 72.39) (end 173.075 70.765) (width 0.25) (layer "F.Cu") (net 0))
 (segment (start 144.78 118.11) (end 166.37 118.11) (width 0.25) (layer "F.Cu") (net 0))
 (segment (start 138.43 77.47) (end 137.16 76.2) (width 0.25) (layer "F.Cu") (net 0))
 (segment (start 142.24 77.47) (end 138.43 77.47) (width 0.25) (layer "F.Cu") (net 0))
 (segment (start 121.92 85.09) (end 121.92 73.66) (width 0.25) (layer "F.Cu") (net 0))
 (segment (start 173.075 70.765) (end 168.91 66.6) (width 0.25) (layer "F.Cu") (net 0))
 (segment (start 163.83 110.49) (end 168.91 105.41) (width 0.25) (layer "F.Cu") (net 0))
 (via (at 130.81 68.58) (size 0.8) (drill 0.4) (layers "F.Cu" "B.Cu") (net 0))
 (via (at 138.43 82.55) (size 0.8) (drill 0.4) (layers "F.Cu" "B.Cu") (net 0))
 (via (at 137.16 81.28) (size 0.8) (drill 0.4) (layers "F.Cu" "B.Cu") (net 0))
 (via (at 133.35 81.28) (size 0.8) (drill 0.4) (layers "F.Cu" "B.Cu") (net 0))
 (via (at 168.91 74.93) (size 0.8) (drill 0.4) (layers "F.Cu" "B.Cu") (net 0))
 (via (at 135.89 82.55) (size 0.8) (drill 0.4) (layers "F.Cu" "B.Cu") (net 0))
 (via (at 171.45 72.39) (size 0.8) (drill 0.4) (layers "F.Cu" "B.Cu") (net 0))
 (via (at 134.62 85.09) (size 0.8) (drill 0.4) (layers "F.Cu" "B.Cu") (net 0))
 (segment (start 130.81 73.66) (end 130.81 68.58) (width 0.25) (layer "B.Cu") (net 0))
 (segment (start 137.16 83.82) (end 135.89 83.82) (width 0.25) (layer "B.Cu") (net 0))
 (segment (start 135.89 82.55) (end 137.16 81.28) (width 0.25) (layer "B.Cu") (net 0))
 (segment (start 168.91 74.93) (end 171.45 72.39) (width 0.25) (layer "B.Cu") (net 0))
 (segment (start 138.43 82.55) (end 137.16 83.82) (width 0.25) (layer "B.Cu") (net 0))
 (segment (start 134.62 85.09) (end 130.81 81.28) (width 0.25) (layer "B.Cu") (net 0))
 (segment (start 135.89 83.82) (end 133.35 81.28) (width 0.25) (layer "B.Cu") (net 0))
 (segment (start 130.81 81.28) (end 130.81 73.66) (width 0.25) (layer "B.Cu") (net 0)))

